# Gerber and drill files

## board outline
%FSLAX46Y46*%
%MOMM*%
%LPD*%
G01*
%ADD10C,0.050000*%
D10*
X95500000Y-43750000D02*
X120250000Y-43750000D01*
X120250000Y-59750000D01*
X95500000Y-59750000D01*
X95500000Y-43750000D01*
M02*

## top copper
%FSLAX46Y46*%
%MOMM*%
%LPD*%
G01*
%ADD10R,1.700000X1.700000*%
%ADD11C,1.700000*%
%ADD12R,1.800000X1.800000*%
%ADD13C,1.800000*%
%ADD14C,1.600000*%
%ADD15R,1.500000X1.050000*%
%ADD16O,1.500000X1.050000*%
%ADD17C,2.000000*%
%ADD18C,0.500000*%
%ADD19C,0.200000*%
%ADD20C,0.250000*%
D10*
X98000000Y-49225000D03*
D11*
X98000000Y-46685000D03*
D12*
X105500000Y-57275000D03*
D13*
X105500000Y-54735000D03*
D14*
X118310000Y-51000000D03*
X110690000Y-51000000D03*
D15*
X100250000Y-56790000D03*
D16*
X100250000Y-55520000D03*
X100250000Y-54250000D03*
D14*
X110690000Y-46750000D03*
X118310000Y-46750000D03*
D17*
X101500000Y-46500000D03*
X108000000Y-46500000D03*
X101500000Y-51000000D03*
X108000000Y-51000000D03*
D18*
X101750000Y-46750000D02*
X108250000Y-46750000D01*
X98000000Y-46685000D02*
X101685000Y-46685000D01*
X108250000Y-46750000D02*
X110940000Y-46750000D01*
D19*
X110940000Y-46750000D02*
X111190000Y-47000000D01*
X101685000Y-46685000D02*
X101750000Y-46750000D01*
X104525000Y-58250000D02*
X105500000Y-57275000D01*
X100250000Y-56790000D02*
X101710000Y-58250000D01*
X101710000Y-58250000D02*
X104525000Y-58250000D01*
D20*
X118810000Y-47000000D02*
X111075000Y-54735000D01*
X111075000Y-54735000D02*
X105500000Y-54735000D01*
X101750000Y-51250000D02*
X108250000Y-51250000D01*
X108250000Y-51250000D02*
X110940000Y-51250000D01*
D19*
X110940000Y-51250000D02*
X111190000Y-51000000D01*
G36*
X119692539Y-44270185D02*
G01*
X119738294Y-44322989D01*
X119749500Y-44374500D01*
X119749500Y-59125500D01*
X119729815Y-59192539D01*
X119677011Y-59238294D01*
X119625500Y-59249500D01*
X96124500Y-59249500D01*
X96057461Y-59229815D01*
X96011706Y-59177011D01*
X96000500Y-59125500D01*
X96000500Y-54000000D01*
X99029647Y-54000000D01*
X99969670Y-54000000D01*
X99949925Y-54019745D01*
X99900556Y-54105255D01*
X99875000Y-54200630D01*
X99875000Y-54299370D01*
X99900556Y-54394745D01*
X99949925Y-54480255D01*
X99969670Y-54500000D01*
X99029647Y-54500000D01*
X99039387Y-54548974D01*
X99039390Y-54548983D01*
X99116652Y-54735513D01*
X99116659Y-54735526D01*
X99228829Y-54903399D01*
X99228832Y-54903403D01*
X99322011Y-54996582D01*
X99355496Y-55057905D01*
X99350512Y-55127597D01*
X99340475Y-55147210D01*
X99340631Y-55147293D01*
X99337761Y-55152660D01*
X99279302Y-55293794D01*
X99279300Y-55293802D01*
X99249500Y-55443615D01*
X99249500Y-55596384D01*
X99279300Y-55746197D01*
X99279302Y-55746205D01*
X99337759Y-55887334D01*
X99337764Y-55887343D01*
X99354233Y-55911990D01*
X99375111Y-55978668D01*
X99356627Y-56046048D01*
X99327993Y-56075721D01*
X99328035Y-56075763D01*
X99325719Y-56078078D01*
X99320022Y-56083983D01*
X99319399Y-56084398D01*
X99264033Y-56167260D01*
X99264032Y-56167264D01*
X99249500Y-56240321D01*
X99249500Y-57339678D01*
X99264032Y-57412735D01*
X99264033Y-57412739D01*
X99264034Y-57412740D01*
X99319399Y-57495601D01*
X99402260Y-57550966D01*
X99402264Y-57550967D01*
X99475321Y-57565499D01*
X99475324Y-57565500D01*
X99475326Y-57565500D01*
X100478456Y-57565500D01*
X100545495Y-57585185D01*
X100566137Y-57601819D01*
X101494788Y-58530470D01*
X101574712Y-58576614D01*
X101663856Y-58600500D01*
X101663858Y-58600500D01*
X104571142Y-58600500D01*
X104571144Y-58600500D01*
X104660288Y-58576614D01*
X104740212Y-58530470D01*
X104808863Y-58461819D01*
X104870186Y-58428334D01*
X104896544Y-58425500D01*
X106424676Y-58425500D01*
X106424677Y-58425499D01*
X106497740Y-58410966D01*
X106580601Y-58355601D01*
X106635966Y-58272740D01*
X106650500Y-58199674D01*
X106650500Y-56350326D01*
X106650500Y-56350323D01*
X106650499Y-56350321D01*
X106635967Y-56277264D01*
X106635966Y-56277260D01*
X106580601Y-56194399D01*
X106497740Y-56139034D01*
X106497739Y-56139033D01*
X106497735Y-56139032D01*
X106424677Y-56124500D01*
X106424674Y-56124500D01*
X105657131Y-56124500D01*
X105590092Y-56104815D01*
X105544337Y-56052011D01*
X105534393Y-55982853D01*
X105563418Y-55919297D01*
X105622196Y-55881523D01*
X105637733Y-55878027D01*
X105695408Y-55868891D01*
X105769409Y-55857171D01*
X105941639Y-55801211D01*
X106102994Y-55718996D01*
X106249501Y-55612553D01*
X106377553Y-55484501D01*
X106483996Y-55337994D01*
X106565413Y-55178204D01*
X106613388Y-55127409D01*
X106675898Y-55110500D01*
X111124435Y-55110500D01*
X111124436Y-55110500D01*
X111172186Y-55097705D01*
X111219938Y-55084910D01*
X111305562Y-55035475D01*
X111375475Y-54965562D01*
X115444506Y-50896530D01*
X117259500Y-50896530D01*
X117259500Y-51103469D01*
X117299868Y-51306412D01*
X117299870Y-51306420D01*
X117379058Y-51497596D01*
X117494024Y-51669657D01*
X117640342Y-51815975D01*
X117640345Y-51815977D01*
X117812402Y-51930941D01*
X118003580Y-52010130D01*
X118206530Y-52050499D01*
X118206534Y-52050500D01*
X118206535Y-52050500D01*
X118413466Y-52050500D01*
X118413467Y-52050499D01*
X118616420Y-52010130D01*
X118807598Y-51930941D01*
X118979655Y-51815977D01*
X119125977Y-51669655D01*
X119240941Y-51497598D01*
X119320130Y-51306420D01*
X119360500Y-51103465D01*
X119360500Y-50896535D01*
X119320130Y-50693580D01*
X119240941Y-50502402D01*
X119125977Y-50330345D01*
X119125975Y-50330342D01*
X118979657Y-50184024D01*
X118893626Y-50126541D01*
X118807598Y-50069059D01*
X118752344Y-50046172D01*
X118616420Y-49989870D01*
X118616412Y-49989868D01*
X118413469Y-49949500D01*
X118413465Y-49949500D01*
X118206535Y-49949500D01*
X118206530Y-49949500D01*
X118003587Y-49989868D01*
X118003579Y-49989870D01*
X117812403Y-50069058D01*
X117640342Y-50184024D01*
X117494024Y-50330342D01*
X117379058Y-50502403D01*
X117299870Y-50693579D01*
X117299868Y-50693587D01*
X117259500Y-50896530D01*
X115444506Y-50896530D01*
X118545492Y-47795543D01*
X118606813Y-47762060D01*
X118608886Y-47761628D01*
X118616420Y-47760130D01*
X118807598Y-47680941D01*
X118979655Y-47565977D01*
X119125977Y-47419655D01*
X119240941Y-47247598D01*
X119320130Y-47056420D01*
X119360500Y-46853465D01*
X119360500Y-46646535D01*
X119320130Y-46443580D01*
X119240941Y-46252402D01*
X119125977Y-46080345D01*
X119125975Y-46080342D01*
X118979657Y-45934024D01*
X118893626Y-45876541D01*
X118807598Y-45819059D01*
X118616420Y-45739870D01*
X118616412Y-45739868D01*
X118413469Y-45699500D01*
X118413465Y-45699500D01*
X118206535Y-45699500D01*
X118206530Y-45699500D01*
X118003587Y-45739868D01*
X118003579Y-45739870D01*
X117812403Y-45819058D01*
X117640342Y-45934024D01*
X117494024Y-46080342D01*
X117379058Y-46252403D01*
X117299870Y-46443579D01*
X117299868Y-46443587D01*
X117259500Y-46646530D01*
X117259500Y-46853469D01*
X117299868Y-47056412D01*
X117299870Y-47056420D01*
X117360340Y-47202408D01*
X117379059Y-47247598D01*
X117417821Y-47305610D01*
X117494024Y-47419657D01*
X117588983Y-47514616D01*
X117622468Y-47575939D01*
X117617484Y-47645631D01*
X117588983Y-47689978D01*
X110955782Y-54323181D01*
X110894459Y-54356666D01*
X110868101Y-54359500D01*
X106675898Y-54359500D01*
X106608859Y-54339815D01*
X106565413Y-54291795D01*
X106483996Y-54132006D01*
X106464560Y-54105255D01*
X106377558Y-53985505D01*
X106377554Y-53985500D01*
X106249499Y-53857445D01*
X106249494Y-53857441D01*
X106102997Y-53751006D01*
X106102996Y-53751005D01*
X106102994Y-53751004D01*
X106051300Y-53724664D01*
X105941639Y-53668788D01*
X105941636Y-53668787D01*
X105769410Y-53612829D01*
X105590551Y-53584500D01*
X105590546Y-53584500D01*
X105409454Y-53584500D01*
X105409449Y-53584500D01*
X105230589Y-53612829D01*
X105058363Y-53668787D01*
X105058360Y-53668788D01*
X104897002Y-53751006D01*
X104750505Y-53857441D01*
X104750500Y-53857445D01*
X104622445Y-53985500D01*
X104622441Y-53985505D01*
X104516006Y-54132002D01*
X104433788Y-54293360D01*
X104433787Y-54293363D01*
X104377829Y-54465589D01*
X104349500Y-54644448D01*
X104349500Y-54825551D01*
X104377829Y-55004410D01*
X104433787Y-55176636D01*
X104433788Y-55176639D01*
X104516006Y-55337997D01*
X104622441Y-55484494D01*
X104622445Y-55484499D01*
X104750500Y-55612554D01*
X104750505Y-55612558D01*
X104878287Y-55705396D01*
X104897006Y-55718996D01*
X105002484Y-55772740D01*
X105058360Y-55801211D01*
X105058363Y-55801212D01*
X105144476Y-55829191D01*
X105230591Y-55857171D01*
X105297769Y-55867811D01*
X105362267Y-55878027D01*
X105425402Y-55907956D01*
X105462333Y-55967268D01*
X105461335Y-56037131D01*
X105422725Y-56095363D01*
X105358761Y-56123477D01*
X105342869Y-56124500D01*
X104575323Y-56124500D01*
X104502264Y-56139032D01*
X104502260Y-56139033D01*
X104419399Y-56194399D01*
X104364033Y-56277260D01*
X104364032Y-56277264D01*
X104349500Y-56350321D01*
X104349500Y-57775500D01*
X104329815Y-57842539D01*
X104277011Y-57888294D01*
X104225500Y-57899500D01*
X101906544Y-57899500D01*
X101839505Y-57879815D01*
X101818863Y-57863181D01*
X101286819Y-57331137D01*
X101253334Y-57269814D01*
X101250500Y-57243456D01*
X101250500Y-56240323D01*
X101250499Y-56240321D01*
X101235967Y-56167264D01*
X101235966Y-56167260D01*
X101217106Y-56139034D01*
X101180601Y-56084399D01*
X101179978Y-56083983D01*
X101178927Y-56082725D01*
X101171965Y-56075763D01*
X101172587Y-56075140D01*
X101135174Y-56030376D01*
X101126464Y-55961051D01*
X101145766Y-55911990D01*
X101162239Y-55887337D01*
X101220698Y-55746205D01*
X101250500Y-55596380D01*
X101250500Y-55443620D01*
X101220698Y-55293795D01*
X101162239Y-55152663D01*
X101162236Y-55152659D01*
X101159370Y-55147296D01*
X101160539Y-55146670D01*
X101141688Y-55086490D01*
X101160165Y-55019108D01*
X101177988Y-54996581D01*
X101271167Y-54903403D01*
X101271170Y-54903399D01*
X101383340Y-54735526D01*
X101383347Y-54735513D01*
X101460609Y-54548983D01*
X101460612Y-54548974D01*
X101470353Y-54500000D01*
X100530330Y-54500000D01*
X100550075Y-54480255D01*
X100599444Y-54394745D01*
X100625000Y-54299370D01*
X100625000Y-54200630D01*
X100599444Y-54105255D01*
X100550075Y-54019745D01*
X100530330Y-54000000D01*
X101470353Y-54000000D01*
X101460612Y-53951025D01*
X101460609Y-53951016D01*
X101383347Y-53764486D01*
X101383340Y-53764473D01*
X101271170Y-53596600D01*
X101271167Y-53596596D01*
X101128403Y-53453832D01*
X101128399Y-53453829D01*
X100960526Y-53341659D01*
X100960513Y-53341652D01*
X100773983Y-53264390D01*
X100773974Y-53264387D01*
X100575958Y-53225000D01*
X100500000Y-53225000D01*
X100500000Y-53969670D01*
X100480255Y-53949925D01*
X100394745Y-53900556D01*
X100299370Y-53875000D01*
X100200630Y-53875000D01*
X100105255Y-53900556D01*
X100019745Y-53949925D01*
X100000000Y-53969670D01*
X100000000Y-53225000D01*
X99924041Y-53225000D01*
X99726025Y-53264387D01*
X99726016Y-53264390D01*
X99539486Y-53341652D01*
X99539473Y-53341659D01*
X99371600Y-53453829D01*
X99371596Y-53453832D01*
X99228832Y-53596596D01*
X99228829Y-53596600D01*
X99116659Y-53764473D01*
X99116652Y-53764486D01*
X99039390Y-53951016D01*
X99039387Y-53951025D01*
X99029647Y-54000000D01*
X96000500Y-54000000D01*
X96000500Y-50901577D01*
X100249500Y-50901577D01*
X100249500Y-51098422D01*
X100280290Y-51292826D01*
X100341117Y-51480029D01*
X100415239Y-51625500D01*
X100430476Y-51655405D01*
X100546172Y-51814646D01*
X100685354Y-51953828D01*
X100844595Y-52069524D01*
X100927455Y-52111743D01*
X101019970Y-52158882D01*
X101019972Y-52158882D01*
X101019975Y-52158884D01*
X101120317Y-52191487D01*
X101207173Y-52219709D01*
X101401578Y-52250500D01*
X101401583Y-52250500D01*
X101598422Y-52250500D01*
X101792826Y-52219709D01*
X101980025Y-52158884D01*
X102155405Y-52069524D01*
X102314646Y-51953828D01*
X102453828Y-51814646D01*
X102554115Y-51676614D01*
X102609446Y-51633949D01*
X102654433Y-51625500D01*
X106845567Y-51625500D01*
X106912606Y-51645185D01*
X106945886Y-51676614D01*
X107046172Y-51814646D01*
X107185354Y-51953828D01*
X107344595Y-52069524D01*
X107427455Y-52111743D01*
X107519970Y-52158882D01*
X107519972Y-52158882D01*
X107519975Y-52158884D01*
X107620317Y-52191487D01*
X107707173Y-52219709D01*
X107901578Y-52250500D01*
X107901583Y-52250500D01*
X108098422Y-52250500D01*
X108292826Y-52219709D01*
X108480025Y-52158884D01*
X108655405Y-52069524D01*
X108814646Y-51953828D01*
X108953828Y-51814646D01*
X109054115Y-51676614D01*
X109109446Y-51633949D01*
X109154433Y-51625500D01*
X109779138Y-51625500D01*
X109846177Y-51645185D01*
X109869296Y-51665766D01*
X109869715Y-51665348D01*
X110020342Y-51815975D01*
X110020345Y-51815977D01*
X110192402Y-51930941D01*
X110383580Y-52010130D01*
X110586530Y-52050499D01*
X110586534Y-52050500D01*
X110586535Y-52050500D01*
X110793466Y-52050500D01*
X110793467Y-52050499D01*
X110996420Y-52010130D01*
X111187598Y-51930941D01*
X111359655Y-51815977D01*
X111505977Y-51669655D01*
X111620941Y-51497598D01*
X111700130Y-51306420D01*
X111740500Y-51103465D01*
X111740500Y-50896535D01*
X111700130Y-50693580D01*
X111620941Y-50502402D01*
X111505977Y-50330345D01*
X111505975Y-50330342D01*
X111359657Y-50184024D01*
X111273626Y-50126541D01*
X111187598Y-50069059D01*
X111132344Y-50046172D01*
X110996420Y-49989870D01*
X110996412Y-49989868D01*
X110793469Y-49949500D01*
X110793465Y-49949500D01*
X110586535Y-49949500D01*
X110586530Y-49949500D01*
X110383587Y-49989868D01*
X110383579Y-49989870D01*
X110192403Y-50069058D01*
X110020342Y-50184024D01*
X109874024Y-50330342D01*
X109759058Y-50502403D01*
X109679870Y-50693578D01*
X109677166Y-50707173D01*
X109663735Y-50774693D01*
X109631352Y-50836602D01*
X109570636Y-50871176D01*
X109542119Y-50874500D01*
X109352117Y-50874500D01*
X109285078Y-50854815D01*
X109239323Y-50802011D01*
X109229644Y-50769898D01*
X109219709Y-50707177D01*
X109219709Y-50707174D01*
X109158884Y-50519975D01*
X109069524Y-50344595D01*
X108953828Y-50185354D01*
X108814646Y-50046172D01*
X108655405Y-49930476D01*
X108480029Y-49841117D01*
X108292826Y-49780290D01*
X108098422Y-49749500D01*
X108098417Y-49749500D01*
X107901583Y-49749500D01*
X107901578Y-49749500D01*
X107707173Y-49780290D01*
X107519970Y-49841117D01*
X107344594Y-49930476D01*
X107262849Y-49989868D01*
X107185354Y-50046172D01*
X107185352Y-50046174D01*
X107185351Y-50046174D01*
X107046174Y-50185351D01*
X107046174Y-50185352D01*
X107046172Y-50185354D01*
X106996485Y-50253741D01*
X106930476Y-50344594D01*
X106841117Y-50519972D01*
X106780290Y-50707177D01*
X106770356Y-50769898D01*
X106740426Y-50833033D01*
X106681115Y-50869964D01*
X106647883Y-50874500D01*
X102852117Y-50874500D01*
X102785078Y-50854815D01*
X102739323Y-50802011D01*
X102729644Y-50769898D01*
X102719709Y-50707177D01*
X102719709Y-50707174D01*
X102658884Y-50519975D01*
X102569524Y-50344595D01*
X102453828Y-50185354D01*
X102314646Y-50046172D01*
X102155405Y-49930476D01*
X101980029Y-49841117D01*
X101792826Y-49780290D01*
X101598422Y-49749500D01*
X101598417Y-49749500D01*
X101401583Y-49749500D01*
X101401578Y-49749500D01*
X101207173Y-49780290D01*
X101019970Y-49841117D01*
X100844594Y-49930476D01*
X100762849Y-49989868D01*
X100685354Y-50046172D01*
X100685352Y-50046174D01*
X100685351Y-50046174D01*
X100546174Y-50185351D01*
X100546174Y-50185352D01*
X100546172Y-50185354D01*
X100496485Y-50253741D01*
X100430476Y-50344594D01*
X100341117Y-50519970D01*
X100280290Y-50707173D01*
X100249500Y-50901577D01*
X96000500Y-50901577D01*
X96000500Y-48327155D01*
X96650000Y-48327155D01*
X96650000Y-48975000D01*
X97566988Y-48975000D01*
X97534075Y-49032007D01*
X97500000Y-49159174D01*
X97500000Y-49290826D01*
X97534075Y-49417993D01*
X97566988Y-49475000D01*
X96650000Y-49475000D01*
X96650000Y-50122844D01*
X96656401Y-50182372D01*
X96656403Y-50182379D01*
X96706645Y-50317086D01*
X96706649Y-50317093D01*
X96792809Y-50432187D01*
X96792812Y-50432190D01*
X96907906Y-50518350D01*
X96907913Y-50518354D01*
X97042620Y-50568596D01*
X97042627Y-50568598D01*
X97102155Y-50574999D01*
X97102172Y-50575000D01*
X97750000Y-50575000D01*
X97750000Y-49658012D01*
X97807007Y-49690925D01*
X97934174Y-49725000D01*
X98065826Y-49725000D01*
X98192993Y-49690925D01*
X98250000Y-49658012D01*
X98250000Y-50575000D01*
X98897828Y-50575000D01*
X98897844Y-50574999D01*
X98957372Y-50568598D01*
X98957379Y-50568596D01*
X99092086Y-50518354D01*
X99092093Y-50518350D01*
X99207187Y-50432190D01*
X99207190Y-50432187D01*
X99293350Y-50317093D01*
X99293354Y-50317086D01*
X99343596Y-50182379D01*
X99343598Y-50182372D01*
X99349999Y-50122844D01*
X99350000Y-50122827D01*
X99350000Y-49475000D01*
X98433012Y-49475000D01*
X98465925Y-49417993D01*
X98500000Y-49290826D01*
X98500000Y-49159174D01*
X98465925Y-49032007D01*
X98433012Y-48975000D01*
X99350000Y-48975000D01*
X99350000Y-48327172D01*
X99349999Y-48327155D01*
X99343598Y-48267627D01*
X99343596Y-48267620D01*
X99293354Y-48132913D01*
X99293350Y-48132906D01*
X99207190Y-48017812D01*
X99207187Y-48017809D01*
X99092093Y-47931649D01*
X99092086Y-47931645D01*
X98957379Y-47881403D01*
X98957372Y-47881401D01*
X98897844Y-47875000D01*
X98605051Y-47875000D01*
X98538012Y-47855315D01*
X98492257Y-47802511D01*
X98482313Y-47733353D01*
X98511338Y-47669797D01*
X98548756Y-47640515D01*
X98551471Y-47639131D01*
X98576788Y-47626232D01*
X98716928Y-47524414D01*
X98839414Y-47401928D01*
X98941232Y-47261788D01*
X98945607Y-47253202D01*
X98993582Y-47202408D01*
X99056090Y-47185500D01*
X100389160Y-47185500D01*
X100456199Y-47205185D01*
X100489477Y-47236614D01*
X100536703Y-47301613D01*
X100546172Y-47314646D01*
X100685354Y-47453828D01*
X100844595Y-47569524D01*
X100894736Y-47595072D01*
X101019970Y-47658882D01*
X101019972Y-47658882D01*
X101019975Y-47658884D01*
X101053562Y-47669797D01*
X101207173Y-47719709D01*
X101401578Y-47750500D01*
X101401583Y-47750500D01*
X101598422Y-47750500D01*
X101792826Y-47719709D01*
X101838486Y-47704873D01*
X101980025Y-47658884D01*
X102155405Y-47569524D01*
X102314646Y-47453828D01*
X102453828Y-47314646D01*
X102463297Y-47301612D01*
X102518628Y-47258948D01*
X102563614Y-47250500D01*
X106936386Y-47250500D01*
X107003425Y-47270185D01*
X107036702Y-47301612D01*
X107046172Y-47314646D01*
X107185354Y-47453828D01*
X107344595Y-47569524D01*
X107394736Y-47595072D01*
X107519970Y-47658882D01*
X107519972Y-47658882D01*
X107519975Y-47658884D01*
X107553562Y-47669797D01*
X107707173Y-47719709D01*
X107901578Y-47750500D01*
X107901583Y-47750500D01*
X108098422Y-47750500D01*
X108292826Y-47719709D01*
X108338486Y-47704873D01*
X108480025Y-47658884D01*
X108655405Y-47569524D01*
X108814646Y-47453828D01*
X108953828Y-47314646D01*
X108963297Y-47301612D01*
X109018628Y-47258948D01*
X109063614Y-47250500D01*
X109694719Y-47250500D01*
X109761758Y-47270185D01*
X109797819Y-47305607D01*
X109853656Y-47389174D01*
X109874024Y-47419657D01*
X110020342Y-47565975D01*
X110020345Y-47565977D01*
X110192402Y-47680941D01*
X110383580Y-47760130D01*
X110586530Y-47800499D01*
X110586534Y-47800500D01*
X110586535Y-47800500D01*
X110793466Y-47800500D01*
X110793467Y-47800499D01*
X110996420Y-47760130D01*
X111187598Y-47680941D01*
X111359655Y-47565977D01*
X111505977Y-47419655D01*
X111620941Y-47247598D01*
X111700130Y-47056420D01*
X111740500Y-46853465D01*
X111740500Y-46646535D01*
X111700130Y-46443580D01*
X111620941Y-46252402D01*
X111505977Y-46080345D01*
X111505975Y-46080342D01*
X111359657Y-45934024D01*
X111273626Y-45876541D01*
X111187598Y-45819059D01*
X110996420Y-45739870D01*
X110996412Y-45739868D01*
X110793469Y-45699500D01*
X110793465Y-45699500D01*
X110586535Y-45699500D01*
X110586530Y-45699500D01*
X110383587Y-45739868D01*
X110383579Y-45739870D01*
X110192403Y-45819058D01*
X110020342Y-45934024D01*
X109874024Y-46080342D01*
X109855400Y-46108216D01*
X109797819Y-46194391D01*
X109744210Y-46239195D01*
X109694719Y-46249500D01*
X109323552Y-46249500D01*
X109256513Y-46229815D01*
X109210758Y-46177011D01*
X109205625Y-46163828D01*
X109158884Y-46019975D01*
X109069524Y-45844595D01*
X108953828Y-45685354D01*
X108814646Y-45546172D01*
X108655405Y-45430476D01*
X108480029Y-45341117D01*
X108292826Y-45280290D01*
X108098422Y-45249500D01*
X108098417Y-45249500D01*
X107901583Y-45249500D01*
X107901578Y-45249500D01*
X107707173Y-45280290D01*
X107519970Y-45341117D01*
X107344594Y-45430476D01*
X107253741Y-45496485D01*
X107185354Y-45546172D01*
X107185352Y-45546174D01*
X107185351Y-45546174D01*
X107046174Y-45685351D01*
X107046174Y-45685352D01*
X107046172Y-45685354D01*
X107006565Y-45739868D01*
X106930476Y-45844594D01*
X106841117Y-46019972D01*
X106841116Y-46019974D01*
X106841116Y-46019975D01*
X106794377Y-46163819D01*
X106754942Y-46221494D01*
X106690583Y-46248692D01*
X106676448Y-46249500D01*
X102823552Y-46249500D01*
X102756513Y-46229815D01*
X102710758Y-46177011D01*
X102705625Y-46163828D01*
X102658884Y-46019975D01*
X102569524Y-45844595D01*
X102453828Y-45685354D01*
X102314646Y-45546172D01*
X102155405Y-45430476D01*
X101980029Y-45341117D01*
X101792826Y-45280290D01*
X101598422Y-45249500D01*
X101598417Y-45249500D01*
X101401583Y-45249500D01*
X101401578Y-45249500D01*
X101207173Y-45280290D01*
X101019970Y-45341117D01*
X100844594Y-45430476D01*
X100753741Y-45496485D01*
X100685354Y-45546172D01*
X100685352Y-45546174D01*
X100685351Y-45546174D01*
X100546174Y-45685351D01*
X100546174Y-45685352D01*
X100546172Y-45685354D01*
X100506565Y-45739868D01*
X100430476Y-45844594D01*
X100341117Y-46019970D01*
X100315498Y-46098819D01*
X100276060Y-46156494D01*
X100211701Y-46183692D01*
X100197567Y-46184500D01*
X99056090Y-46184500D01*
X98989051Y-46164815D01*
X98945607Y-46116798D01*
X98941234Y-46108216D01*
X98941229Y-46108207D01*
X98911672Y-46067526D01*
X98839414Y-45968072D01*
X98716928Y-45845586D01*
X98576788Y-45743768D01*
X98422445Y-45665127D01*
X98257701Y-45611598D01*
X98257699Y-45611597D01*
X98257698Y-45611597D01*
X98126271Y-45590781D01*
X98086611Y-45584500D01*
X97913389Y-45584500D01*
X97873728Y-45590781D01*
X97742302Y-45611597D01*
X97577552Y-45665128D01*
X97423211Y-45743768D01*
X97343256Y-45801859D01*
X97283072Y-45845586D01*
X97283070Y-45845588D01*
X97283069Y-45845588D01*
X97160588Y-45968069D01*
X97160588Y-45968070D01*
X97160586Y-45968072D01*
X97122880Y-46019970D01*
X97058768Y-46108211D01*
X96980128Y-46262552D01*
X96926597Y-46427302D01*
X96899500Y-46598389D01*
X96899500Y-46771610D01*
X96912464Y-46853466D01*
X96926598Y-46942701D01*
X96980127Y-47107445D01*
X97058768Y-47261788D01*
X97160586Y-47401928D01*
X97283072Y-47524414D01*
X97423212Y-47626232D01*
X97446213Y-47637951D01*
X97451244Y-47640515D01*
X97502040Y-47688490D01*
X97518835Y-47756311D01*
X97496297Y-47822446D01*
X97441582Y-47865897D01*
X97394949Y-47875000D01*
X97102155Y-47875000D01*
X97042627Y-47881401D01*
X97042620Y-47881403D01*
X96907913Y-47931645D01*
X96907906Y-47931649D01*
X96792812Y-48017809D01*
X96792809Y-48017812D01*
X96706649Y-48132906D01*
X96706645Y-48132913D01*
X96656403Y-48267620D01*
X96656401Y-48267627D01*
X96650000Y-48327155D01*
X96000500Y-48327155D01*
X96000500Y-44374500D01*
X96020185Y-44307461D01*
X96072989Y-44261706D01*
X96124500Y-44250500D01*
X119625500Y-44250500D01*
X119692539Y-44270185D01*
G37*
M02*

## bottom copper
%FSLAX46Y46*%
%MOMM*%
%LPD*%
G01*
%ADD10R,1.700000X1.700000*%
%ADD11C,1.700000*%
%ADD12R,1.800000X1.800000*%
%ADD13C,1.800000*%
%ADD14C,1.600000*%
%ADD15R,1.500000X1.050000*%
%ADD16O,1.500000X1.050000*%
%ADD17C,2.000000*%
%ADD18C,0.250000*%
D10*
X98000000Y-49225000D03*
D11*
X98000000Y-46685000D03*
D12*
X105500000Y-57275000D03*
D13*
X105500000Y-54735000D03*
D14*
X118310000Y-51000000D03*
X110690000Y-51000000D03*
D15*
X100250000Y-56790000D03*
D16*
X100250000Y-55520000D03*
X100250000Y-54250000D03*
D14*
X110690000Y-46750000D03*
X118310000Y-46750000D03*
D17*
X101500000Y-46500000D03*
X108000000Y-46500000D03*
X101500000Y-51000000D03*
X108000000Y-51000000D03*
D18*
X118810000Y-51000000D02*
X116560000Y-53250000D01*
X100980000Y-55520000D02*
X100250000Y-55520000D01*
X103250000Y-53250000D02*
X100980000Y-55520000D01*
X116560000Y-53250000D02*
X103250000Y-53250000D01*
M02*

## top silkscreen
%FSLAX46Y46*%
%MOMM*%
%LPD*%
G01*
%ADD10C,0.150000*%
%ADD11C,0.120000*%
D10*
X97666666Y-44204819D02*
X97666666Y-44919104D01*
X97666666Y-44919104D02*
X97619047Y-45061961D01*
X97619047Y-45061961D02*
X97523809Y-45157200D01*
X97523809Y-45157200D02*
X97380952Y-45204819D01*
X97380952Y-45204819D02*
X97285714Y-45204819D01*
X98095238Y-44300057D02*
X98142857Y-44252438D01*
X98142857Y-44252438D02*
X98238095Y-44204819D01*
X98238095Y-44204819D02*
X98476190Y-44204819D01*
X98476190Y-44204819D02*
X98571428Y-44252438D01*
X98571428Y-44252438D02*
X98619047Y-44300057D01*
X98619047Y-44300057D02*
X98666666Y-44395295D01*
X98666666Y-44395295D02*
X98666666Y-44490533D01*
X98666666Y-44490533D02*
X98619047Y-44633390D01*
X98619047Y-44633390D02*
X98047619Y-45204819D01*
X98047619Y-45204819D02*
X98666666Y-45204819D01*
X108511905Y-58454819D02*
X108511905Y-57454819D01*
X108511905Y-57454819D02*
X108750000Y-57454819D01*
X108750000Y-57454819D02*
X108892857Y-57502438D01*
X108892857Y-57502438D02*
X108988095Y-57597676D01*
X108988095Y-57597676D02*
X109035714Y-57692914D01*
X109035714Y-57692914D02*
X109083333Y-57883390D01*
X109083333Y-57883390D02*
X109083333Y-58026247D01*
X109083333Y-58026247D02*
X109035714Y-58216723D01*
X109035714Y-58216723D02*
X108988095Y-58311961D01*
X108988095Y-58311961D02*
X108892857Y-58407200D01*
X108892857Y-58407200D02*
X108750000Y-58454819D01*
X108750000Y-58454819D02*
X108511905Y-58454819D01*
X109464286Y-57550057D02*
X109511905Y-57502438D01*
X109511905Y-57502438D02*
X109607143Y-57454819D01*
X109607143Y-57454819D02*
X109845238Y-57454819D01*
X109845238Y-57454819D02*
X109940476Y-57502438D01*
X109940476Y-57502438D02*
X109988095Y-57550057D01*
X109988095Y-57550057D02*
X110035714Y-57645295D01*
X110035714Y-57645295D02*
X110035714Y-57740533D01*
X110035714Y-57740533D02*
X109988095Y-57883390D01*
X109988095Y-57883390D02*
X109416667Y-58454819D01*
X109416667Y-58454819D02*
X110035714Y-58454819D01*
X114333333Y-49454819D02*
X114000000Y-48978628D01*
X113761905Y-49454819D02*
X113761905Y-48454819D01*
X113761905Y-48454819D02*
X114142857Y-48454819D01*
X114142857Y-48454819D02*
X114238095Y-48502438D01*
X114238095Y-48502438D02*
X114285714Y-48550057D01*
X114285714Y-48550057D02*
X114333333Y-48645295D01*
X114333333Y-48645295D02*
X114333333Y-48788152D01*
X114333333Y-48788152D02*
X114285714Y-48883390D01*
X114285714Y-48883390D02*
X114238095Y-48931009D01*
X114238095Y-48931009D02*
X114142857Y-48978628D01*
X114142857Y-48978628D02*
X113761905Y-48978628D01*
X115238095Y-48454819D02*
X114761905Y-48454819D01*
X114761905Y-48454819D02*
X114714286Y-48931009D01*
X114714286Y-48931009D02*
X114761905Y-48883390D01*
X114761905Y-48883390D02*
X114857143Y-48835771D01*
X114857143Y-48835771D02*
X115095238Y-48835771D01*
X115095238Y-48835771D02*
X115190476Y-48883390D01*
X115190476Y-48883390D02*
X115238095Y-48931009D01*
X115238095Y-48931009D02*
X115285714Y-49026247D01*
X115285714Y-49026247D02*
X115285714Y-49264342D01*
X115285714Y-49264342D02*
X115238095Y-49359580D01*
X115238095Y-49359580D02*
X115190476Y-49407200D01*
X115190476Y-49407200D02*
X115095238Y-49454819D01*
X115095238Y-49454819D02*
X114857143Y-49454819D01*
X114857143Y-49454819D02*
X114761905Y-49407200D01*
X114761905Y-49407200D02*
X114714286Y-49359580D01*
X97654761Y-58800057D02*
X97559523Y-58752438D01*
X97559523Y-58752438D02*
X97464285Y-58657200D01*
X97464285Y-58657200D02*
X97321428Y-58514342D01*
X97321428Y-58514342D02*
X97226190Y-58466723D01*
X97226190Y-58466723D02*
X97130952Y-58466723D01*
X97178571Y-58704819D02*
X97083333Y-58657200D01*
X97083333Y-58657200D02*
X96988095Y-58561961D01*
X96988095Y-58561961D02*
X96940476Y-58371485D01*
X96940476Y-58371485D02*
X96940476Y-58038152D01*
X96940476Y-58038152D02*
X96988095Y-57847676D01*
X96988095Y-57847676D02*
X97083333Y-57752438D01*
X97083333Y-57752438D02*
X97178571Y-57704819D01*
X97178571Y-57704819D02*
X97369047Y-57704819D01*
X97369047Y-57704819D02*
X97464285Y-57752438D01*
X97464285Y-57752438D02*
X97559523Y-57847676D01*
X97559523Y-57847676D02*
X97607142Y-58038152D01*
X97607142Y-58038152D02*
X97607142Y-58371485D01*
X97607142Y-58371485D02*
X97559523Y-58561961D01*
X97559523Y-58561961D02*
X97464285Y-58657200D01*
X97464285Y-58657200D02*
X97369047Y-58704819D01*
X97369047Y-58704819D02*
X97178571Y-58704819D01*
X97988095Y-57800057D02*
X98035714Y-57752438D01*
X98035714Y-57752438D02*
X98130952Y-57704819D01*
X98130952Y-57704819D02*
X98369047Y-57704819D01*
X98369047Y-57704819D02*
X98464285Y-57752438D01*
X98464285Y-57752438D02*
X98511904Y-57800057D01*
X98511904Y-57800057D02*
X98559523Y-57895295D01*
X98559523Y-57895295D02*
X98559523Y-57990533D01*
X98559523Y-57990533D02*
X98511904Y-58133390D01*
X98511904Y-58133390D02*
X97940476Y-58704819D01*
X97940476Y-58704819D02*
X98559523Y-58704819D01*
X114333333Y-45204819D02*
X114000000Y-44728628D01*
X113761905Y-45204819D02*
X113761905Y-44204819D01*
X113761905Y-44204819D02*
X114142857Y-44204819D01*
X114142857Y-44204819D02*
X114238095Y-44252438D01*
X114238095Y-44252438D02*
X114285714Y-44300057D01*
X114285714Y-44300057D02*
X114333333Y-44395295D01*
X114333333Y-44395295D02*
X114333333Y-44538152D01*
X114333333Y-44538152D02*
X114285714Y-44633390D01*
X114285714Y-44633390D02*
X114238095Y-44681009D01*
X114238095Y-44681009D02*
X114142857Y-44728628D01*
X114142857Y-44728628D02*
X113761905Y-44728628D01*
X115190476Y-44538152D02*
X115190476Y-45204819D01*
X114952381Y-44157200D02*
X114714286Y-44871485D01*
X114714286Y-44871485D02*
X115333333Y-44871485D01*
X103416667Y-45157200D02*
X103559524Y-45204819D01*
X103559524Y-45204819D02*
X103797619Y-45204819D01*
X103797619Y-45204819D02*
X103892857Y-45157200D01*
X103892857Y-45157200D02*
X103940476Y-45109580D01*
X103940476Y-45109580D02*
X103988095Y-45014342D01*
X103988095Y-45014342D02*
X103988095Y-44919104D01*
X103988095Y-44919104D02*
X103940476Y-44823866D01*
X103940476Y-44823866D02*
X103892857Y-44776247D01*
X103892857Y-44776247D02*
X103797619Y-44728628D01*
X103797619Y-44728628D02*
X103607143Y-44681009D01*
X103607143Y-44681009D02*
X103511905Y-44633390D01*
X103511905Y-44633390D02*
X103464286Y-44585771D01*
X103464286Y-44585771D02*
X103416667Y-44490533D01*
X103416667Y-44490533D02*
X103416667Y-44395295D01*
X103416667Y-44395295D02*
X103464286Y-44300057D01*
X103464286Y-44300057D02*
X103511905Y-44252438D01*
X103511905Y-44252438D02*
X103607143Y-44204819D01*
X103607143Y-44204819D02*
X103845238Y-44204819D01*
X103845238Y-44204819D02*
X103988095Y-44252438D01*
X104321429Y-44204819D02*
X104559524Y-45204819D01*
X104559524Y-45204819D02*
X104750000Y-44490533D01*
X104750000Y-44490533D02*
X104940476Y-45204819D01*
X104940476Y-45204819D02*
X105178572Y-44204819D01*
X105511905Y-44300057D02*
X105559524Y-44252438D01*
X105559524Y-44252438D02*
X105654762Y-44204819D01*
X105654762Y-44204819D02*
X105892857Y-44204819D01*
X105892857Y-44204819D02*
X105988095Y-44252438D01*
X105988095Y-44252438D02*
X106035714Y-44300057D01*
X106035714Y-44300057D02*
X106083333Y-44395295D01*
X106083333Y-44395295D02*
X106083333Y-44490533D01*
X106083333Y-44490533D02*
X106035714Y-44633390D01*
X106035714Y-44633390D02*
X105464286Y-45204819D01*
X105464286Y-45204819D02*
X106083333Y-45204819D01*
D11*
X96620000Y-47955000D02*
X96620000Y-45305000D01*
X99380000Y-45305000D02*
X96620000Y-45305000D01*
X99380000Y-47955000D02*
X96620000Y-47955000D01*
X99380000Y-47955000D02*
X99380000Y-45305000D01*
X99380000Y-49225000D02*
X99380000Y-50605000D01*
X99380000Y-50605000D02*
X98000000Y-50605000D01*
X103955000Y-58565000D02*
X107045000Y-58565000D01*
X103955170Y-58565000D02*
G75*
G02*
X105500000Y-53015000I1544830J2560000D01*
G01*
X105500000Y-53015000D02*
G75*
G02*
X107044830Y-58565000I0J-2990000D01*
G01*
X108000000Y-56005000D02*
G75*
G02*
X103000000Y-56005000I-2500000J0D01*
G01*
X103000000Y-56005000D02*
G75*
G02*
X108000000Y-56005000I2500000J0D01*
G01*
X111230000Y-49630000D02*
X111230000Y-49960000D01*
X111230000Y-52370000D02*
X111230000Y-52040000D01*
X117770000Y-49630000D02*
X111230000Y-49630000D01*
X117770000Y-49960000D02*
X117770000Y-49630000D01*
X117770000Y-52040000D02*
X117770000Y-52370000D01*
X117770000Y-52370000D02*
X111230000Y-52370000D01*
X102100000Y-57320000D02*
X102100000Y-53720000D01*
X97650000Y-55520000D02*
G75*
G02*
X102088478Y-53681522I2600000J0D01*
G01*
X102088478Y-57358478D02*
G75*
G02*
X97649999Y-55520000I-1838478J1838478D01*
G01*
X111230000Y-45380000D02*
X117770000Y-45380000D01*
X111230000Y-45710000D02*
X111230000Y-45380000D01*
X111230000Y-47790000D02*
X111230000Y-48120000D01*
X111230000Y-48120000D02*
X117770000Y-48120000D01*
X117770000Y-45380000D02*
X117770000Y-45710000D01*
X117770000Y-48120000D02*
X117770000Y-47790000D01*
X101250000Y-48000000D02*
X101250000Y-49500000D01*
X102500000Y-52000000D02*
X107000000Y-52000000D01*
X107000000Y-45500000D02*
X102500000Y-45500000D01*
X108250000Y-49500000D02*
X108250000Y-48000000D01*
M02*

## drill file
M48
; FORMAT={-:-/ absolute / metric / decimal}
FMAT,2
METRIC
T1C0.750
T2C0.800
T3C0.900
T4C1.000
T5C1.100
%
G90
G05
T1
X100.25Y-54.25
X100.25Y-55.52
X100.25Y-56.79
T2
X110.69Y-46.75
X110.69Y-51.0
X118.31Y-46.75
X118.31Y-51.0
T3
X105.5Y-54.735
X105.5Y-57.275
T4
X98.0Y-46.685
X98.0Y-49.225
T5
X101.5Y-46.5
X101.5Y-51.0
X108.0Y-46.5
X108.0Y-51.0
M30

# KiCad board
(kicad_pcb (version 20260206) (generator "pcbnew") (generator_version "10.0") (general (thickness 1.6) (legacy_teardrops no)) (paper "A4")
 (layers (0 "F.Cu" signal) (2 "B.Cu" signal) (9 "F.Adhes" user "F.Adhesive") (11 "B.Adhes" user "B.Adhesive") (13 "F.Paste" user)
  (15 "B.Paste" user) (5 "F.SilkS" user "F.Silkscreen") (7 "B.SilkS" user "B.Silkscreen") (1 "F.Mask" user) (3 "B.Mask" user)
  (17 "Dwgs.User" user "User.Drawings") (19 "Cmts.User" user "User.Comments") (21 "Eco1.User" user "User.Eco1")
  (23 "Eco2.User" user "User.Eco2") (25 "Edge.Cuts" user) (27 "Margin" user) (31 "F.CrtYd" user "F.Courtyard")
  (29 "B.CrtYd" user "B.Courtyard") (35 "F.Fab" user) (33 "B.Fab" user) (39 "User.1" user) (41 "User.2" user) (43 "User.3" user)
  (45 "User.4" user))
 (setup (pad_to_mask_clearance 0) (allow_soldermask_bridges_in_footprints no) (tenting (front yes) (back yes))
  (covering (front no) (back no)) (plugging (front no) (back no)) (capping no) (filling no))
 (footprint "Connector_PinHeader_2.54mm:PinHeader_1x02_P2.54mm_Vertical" (layer "F.Cu") (at 98 49.225 180)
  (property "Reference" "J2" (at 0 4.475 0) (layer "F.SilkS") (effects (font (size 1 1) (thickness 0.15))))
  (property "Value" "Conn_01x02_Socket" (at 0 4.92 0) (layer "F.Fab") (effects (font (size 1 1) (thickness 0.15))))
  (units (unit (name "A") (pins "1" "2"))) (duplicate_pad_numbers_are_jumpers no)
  (fp_line (start 1.38 1.27) (end 1.38 3.92) (stroke (width 0.12) (type solid)) (layer "F.SilkS"))
  (fp_line (start -1.38 3.92) (end 1.38 3.92) (stroke (width 0.12) (type solid)) (layer "F.SilkS"))
  (fp_line (start -1.38 1.27) (end 1.38 1.27) (stroke (width 0.12) (type solid)) (layer "F.SilkS"))
  (fp_line (start -1.38 1.27) (end -1.38 3.92) (stroke (width 0.12) (type solid)) (layer "F.SilkS"))
  (fp_line (start -1.38 0) (end -1.38 -1.38) (stroke (width 0.12) (type solid)) (layer "F.SilkS"))
  (fp_line (start -1.38 -1.38) (end 0 -1.38) (stroke (width 0.12) (type solid)) (layer "F.SilkS"))
  (pad "1" thru_hole rect (at 0 0 180) (size 1.7 1.7) (drill 1) (layers "*.Cu" "*.Mask") (remove_unused_layers no) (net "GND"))
  (pad "2" thru_hole circle (at 0 2.54 180) (size 1.7 1.7) (drill 1) (layers "*.Cu" "*.Mask") (remove_unused_layers no) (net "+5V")))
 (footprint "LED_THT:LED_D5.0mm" (layer "F.Cu") (at 105.5 57.275 90)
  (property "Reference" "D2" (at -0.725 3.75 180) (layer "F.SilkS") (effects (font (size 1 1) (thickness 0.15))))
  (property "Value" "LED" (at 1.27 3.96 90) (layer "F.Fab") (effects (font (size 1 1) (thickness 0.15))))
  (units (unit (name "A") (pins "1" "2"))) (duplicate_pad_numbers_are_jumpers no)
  (fp_line (start -1.29 -1.545) (end -1.29 1.545) (stroke (width 0.12) (type solid)) (layer "F.SilkS"))
  (fp_arc (start -1.29 -1.54483) (mid 2.071779 -2.880495) (end 4.26 0) (stroke (width 0.12) (type solid)) (layer "F.SilkS"))
  (fp_arc (start 4.26 0) (mid 2.071779 2.880495) (end -1.29 1.54483) (stroke (width 0.12) (type solid)) (layer "F.SilkS"))
  (fp_circle (center 1.27 0) (end 3.77 0) (stroke (width 0.12) (type solid)) (fill no) (layer "F.SilkS"))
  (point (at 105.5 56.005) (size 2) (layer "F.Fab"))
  (pad "1" thru_hole rect (at 0 0 90) (size 1.8 1.8) (drill 0.9) (layers "*.Cu" "*.Mask") (remove_unused_layers no) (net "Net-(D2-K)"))
  (pad "2" thru_hole circle (at 2.54 0 90) (size 1.8 1.8) (drill 0.9) (layers "*.Cu" "*.Mask") (remove_unused_layers no) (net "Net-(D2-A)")))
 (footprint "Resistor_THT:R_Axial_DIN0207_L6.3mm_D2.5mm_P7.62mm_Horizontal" (layer "F.Cu") (at 118.31 51 180)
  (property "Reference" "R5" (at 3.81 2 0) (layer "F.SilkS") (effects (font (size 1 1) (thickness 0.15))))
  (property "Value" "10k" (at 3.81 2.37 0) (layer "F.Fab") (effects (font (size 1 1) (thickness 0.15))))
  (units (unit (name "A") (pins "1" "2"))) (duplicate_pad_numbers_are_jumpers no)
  (fp_line (start 7.08 1.37) (end 7.08 1.04) (stroke (width 0.12) (type solid)) (layer "F.SilkS"))
  (fp_line (start 7.08 -1.37) (end 7.08 -1.04) (stroke (width 0.12) (type solid)) (layer "F.SilkS"))
  (fp_line (start 0.54 1.37) (end 7.08 1.37) (stroke (width 0.12) (type solid)) (layer "F.SilkS"))
  (fp_line (start 0.54 1.04) (end 0.54 1.37) (stroke (width 0.12) (type solid)) (layer "F.SilkS"))
  (fp_line (start 0.54 -1.04) (end 0.54 -1.37) (stroke (width 0.12) (type solid)) (layer "F.SilkS"))
  (fp_line (start 0.54 -1.37) (end 7.08 -1.37) (stroke (width 0.12) (type solid)) (layer "F.SilkS"))
  (pad "1" thru_hole circle (at 0 0 180) (size 1.6 1.6) (drill 0.8) (layers "*.Cu" "*.Mask") (remove_unused_layers no) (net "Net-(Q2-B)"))
  (pad "2" thru_hole circle (at 7.62 0 180) (size 1.6 1.6) (drill 0.8) (layers "*.Cu" "*.Mask") (remove_unused_layers no)
   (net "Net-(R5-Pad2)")))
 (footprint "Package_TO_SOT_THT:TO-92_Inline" (layer "F.Cu") (at 100.25 56.79 90)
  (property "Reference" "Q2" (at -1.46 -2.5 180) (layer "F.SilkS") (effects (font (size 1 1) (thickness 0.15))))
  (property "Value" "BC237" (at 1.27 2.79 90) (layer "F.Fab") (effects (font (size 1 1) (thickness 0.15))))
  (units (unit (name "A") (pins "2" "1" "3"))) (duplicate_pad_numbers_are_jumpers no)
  (fp_line (start -0.53 1.85) (end 3.07 1.85) (stroke (width 0.12) (type solid)) (layer "F.SilkS"))
  (fp_arc (start 1.27 -2.6) (mid 3.672087 -0.994977) (end 3.108478 1.838478) (stroke (width 0.12) (type solid)) (layer "F.SilkS"))
  (fp_arc (start -0.568478 1.838478) (mid -1.132087 -0.994977) (end 1.27 -2.6) (stroke (width 0.12) (type solid)) (layer "F.SilkS"))
  (pad "1" thru_hole rect (at 0 0 90) (size 1.05 1.5) (drill 0.75) (layers "*.Cu" "*.Mask") (remove_unused_layers no) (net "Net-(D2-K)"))
  (pad "2" thru_hole oval (at 1.27 0 90) (size 1.05 1.5) (drill 0.75) (layers "*.Cu" "*.Mask") (remove_unused_layers no) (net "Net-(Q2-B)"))
  (pad "3" thru_hole oval (at 2.54 0 90) (size 1.05 1.5) (drill 0.75) (layers "*.Cu" "*.Mask") (remove_unused_layers no) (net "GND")))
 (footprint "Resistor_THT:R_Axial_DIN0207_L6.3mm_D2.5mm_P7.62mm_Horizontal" (layer "F.Cu") (at 110.69 46.75)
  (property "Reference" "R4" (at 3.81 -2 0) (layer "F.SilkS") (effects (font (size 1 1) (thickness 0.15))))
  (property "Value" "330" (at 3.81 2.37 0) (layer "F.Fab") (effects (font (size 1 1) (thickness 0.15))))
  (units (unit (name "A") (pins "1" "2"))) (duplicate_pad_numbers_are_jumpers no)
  (fp_line (start 0.54 -1.37) (end 7.08 -1.37) (stroke (width 0.12) (type solid)) (layer "F.SilkS"))
  (fp_line (start 0.54 -1.04) (end 0.54 -1.37) (stroke (width 0.12) (type solid)) (layer "F.SilkS"))
  (fp_line (start 0.54 1.04) (end 0.54 1.37) (stroke (width 0.12) (type solid)) (layer "F.SilkS"))
  (fp_line (start 0.54 1.37) (end 7.08 1.37) (stroke (width 0.12) (type solid)) (layer "F.SilkS"))
  (fp_line (start 7.08 -1.37) (end 7.08 -1.04) (stroke (width 0.12) (type solid)) (layer "F.SilkS"))
  (fp_line (start 7.08 1.37) (end 7.08 1.04) (stroke (width 0.12) (type solid)) (layer "F.SilkS"))
  (pad "1" thru_hole circle (at 0 0) (size 1.6 1.6) (drill 0.8) (layers "*.Cu" "*.Mask") (remove_unused_layers no) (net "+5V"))
  (pad "2" thru_hole circle (at 7.62 0) (size 1.6 1.6) (drill 0.8) (layers "*.Cu" "*.Mask") (remove_unused_layers no) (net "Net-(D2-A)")))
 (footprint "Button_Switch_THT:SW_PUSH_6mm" (layer "F.Cu") (at 101.5 46.5)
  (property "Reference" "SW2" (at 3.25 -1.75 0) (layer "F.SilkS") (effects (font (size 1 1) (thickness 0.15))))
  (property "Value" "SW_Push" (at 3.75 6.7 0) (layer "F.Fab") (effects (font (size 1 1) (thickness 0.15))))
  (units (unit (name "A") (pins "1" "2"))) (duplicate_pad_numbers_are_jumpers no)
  (fp_line (start -0.25 1.5) (end -0.25 3) (stroke (width 0.12) (type solid)) (layer "F.SilkS"))
  (fp_line (start 1 5.5) (end 5.5 5.5) (stroke (width 0.12) (type solid)) (layer "F.SilkS"))
  (fp_line (start 5.5 -1) (end 1 -1) (stroke (width 0.12) (type solid)) (layer "F.SilkS"))
  (fp_line (start 6.75 3) (end 6.75 1.5) (stroke (width 0.12) (type solid)) (layer "F.SilkS"))
  (pad "1" thru_hole circle (at 0 0 90) (size 2 2) (drill 1.1) (layers "*.Cu" "*.Mask") (remove_unused_layers no) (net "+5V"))
  (pad "1" thru_hole circle (at 6.5 0 90) (size 2 2) (drill 1.1) (layers "*.Cu" "*.Mask") (remove_unused_layers no) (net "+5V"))
  (pad "2" thru_hole circle (at 0 4.5 90) (size 2 2) (drill 1.1) (layers "*.Cu" "*.Mask") (remove_unused_layers no) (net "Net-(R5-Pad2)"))
  (pad "2" thru_hole circle (at 6.5 4.5 90) (size 2 2) (drill 1.1) (layers "*.Cu" "*.Mask") (remove_unused_layers no) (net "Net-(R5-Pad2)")))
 (gr_rect (start 95.5 43.75) (end 120.25 59.75) (stroke (width 0.05) (type default)) (fill no) (layer "Edge.Cuts"))
 (segment (start 101.75 46.75) (end 108.25 46.75) (width 0.5) (layer "F.Cu") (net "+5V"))
 (segment (start 98 46.685) (end 101.685 46.685) (width 0.5) (layer "F.Cu") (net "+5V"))
 (segment (start 108.25 46.75) (end 110.94 46.75) (width 0.5) (layer "F.Cu") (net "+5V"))
 (segment (start 110.94 46.75) (end 111.19 47) (width 0.2) (layer "F.Cu") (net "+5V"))
 (segment (start 101.685 46.685) (end 101.75 46.75) (width 0.2) (layer "F.Cu") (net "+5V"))
 (segment (start 104.525 58.25) (end 105.5 57.275) (width 0.2) (layer "F.Cu") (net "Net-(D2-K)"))
 (segment (start 100.25 56.79) (end 101.71 58.25) (width 0.2) (layer "F.Cu") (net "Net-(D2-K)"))
 (segment (start 101.71 58.25) (end 104.525 58.25) (width 0.2) (layer "F.Cu") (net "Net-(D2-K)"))
 (segment (start 118.81 47) (end 111.075 54.735) (width 0.25) (layer "F.Cu") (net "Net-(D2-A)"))
 (segment (start 111.075 54.735) (end 105.5 54.735) (width 0.25) (layer "F.Cu") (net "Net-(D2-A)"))
 (segment (start 118.81 51) (end 116.56 53.25) (width 0.25) (layer "B.Cu") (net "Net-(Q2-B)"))
 (segment (start 100.98 55.52) (end 100.25 55.52) (width 0.25) (layer "B.Cu") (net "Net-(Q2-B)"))
 (segment (start 103.25 53.25) (end 100.98 55.52) (width 0.25) (layer "B.Cu") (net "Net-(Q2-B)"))
 (segment (start 116.56 53.25) (end 103.25 53.25) (width 0.25) (layer "B.Cu") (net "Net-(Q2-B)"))
 (segment (start 101.75 51.25) (end 108.25 51.25) (width 0.25) (layer "F.Cu") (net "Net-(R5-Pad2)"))
 (segment (start 108.25 51.25) (end 110.94 51.25) (width 0.25) (layer "F.Cu") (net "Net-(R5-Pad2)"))
 (segment (start 110.94 51.25) (end 111.19 51) (width 0.2) (layer "F.Cu") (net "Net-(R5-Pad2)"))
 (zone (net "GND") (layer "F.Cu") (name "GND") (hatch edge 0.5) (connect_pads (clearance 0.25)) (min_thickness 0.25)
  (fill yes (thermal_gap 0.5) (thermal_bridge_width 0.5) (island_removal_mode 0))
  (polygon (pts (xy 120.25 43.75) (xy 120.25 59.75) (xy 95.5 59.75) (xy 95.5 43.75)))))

